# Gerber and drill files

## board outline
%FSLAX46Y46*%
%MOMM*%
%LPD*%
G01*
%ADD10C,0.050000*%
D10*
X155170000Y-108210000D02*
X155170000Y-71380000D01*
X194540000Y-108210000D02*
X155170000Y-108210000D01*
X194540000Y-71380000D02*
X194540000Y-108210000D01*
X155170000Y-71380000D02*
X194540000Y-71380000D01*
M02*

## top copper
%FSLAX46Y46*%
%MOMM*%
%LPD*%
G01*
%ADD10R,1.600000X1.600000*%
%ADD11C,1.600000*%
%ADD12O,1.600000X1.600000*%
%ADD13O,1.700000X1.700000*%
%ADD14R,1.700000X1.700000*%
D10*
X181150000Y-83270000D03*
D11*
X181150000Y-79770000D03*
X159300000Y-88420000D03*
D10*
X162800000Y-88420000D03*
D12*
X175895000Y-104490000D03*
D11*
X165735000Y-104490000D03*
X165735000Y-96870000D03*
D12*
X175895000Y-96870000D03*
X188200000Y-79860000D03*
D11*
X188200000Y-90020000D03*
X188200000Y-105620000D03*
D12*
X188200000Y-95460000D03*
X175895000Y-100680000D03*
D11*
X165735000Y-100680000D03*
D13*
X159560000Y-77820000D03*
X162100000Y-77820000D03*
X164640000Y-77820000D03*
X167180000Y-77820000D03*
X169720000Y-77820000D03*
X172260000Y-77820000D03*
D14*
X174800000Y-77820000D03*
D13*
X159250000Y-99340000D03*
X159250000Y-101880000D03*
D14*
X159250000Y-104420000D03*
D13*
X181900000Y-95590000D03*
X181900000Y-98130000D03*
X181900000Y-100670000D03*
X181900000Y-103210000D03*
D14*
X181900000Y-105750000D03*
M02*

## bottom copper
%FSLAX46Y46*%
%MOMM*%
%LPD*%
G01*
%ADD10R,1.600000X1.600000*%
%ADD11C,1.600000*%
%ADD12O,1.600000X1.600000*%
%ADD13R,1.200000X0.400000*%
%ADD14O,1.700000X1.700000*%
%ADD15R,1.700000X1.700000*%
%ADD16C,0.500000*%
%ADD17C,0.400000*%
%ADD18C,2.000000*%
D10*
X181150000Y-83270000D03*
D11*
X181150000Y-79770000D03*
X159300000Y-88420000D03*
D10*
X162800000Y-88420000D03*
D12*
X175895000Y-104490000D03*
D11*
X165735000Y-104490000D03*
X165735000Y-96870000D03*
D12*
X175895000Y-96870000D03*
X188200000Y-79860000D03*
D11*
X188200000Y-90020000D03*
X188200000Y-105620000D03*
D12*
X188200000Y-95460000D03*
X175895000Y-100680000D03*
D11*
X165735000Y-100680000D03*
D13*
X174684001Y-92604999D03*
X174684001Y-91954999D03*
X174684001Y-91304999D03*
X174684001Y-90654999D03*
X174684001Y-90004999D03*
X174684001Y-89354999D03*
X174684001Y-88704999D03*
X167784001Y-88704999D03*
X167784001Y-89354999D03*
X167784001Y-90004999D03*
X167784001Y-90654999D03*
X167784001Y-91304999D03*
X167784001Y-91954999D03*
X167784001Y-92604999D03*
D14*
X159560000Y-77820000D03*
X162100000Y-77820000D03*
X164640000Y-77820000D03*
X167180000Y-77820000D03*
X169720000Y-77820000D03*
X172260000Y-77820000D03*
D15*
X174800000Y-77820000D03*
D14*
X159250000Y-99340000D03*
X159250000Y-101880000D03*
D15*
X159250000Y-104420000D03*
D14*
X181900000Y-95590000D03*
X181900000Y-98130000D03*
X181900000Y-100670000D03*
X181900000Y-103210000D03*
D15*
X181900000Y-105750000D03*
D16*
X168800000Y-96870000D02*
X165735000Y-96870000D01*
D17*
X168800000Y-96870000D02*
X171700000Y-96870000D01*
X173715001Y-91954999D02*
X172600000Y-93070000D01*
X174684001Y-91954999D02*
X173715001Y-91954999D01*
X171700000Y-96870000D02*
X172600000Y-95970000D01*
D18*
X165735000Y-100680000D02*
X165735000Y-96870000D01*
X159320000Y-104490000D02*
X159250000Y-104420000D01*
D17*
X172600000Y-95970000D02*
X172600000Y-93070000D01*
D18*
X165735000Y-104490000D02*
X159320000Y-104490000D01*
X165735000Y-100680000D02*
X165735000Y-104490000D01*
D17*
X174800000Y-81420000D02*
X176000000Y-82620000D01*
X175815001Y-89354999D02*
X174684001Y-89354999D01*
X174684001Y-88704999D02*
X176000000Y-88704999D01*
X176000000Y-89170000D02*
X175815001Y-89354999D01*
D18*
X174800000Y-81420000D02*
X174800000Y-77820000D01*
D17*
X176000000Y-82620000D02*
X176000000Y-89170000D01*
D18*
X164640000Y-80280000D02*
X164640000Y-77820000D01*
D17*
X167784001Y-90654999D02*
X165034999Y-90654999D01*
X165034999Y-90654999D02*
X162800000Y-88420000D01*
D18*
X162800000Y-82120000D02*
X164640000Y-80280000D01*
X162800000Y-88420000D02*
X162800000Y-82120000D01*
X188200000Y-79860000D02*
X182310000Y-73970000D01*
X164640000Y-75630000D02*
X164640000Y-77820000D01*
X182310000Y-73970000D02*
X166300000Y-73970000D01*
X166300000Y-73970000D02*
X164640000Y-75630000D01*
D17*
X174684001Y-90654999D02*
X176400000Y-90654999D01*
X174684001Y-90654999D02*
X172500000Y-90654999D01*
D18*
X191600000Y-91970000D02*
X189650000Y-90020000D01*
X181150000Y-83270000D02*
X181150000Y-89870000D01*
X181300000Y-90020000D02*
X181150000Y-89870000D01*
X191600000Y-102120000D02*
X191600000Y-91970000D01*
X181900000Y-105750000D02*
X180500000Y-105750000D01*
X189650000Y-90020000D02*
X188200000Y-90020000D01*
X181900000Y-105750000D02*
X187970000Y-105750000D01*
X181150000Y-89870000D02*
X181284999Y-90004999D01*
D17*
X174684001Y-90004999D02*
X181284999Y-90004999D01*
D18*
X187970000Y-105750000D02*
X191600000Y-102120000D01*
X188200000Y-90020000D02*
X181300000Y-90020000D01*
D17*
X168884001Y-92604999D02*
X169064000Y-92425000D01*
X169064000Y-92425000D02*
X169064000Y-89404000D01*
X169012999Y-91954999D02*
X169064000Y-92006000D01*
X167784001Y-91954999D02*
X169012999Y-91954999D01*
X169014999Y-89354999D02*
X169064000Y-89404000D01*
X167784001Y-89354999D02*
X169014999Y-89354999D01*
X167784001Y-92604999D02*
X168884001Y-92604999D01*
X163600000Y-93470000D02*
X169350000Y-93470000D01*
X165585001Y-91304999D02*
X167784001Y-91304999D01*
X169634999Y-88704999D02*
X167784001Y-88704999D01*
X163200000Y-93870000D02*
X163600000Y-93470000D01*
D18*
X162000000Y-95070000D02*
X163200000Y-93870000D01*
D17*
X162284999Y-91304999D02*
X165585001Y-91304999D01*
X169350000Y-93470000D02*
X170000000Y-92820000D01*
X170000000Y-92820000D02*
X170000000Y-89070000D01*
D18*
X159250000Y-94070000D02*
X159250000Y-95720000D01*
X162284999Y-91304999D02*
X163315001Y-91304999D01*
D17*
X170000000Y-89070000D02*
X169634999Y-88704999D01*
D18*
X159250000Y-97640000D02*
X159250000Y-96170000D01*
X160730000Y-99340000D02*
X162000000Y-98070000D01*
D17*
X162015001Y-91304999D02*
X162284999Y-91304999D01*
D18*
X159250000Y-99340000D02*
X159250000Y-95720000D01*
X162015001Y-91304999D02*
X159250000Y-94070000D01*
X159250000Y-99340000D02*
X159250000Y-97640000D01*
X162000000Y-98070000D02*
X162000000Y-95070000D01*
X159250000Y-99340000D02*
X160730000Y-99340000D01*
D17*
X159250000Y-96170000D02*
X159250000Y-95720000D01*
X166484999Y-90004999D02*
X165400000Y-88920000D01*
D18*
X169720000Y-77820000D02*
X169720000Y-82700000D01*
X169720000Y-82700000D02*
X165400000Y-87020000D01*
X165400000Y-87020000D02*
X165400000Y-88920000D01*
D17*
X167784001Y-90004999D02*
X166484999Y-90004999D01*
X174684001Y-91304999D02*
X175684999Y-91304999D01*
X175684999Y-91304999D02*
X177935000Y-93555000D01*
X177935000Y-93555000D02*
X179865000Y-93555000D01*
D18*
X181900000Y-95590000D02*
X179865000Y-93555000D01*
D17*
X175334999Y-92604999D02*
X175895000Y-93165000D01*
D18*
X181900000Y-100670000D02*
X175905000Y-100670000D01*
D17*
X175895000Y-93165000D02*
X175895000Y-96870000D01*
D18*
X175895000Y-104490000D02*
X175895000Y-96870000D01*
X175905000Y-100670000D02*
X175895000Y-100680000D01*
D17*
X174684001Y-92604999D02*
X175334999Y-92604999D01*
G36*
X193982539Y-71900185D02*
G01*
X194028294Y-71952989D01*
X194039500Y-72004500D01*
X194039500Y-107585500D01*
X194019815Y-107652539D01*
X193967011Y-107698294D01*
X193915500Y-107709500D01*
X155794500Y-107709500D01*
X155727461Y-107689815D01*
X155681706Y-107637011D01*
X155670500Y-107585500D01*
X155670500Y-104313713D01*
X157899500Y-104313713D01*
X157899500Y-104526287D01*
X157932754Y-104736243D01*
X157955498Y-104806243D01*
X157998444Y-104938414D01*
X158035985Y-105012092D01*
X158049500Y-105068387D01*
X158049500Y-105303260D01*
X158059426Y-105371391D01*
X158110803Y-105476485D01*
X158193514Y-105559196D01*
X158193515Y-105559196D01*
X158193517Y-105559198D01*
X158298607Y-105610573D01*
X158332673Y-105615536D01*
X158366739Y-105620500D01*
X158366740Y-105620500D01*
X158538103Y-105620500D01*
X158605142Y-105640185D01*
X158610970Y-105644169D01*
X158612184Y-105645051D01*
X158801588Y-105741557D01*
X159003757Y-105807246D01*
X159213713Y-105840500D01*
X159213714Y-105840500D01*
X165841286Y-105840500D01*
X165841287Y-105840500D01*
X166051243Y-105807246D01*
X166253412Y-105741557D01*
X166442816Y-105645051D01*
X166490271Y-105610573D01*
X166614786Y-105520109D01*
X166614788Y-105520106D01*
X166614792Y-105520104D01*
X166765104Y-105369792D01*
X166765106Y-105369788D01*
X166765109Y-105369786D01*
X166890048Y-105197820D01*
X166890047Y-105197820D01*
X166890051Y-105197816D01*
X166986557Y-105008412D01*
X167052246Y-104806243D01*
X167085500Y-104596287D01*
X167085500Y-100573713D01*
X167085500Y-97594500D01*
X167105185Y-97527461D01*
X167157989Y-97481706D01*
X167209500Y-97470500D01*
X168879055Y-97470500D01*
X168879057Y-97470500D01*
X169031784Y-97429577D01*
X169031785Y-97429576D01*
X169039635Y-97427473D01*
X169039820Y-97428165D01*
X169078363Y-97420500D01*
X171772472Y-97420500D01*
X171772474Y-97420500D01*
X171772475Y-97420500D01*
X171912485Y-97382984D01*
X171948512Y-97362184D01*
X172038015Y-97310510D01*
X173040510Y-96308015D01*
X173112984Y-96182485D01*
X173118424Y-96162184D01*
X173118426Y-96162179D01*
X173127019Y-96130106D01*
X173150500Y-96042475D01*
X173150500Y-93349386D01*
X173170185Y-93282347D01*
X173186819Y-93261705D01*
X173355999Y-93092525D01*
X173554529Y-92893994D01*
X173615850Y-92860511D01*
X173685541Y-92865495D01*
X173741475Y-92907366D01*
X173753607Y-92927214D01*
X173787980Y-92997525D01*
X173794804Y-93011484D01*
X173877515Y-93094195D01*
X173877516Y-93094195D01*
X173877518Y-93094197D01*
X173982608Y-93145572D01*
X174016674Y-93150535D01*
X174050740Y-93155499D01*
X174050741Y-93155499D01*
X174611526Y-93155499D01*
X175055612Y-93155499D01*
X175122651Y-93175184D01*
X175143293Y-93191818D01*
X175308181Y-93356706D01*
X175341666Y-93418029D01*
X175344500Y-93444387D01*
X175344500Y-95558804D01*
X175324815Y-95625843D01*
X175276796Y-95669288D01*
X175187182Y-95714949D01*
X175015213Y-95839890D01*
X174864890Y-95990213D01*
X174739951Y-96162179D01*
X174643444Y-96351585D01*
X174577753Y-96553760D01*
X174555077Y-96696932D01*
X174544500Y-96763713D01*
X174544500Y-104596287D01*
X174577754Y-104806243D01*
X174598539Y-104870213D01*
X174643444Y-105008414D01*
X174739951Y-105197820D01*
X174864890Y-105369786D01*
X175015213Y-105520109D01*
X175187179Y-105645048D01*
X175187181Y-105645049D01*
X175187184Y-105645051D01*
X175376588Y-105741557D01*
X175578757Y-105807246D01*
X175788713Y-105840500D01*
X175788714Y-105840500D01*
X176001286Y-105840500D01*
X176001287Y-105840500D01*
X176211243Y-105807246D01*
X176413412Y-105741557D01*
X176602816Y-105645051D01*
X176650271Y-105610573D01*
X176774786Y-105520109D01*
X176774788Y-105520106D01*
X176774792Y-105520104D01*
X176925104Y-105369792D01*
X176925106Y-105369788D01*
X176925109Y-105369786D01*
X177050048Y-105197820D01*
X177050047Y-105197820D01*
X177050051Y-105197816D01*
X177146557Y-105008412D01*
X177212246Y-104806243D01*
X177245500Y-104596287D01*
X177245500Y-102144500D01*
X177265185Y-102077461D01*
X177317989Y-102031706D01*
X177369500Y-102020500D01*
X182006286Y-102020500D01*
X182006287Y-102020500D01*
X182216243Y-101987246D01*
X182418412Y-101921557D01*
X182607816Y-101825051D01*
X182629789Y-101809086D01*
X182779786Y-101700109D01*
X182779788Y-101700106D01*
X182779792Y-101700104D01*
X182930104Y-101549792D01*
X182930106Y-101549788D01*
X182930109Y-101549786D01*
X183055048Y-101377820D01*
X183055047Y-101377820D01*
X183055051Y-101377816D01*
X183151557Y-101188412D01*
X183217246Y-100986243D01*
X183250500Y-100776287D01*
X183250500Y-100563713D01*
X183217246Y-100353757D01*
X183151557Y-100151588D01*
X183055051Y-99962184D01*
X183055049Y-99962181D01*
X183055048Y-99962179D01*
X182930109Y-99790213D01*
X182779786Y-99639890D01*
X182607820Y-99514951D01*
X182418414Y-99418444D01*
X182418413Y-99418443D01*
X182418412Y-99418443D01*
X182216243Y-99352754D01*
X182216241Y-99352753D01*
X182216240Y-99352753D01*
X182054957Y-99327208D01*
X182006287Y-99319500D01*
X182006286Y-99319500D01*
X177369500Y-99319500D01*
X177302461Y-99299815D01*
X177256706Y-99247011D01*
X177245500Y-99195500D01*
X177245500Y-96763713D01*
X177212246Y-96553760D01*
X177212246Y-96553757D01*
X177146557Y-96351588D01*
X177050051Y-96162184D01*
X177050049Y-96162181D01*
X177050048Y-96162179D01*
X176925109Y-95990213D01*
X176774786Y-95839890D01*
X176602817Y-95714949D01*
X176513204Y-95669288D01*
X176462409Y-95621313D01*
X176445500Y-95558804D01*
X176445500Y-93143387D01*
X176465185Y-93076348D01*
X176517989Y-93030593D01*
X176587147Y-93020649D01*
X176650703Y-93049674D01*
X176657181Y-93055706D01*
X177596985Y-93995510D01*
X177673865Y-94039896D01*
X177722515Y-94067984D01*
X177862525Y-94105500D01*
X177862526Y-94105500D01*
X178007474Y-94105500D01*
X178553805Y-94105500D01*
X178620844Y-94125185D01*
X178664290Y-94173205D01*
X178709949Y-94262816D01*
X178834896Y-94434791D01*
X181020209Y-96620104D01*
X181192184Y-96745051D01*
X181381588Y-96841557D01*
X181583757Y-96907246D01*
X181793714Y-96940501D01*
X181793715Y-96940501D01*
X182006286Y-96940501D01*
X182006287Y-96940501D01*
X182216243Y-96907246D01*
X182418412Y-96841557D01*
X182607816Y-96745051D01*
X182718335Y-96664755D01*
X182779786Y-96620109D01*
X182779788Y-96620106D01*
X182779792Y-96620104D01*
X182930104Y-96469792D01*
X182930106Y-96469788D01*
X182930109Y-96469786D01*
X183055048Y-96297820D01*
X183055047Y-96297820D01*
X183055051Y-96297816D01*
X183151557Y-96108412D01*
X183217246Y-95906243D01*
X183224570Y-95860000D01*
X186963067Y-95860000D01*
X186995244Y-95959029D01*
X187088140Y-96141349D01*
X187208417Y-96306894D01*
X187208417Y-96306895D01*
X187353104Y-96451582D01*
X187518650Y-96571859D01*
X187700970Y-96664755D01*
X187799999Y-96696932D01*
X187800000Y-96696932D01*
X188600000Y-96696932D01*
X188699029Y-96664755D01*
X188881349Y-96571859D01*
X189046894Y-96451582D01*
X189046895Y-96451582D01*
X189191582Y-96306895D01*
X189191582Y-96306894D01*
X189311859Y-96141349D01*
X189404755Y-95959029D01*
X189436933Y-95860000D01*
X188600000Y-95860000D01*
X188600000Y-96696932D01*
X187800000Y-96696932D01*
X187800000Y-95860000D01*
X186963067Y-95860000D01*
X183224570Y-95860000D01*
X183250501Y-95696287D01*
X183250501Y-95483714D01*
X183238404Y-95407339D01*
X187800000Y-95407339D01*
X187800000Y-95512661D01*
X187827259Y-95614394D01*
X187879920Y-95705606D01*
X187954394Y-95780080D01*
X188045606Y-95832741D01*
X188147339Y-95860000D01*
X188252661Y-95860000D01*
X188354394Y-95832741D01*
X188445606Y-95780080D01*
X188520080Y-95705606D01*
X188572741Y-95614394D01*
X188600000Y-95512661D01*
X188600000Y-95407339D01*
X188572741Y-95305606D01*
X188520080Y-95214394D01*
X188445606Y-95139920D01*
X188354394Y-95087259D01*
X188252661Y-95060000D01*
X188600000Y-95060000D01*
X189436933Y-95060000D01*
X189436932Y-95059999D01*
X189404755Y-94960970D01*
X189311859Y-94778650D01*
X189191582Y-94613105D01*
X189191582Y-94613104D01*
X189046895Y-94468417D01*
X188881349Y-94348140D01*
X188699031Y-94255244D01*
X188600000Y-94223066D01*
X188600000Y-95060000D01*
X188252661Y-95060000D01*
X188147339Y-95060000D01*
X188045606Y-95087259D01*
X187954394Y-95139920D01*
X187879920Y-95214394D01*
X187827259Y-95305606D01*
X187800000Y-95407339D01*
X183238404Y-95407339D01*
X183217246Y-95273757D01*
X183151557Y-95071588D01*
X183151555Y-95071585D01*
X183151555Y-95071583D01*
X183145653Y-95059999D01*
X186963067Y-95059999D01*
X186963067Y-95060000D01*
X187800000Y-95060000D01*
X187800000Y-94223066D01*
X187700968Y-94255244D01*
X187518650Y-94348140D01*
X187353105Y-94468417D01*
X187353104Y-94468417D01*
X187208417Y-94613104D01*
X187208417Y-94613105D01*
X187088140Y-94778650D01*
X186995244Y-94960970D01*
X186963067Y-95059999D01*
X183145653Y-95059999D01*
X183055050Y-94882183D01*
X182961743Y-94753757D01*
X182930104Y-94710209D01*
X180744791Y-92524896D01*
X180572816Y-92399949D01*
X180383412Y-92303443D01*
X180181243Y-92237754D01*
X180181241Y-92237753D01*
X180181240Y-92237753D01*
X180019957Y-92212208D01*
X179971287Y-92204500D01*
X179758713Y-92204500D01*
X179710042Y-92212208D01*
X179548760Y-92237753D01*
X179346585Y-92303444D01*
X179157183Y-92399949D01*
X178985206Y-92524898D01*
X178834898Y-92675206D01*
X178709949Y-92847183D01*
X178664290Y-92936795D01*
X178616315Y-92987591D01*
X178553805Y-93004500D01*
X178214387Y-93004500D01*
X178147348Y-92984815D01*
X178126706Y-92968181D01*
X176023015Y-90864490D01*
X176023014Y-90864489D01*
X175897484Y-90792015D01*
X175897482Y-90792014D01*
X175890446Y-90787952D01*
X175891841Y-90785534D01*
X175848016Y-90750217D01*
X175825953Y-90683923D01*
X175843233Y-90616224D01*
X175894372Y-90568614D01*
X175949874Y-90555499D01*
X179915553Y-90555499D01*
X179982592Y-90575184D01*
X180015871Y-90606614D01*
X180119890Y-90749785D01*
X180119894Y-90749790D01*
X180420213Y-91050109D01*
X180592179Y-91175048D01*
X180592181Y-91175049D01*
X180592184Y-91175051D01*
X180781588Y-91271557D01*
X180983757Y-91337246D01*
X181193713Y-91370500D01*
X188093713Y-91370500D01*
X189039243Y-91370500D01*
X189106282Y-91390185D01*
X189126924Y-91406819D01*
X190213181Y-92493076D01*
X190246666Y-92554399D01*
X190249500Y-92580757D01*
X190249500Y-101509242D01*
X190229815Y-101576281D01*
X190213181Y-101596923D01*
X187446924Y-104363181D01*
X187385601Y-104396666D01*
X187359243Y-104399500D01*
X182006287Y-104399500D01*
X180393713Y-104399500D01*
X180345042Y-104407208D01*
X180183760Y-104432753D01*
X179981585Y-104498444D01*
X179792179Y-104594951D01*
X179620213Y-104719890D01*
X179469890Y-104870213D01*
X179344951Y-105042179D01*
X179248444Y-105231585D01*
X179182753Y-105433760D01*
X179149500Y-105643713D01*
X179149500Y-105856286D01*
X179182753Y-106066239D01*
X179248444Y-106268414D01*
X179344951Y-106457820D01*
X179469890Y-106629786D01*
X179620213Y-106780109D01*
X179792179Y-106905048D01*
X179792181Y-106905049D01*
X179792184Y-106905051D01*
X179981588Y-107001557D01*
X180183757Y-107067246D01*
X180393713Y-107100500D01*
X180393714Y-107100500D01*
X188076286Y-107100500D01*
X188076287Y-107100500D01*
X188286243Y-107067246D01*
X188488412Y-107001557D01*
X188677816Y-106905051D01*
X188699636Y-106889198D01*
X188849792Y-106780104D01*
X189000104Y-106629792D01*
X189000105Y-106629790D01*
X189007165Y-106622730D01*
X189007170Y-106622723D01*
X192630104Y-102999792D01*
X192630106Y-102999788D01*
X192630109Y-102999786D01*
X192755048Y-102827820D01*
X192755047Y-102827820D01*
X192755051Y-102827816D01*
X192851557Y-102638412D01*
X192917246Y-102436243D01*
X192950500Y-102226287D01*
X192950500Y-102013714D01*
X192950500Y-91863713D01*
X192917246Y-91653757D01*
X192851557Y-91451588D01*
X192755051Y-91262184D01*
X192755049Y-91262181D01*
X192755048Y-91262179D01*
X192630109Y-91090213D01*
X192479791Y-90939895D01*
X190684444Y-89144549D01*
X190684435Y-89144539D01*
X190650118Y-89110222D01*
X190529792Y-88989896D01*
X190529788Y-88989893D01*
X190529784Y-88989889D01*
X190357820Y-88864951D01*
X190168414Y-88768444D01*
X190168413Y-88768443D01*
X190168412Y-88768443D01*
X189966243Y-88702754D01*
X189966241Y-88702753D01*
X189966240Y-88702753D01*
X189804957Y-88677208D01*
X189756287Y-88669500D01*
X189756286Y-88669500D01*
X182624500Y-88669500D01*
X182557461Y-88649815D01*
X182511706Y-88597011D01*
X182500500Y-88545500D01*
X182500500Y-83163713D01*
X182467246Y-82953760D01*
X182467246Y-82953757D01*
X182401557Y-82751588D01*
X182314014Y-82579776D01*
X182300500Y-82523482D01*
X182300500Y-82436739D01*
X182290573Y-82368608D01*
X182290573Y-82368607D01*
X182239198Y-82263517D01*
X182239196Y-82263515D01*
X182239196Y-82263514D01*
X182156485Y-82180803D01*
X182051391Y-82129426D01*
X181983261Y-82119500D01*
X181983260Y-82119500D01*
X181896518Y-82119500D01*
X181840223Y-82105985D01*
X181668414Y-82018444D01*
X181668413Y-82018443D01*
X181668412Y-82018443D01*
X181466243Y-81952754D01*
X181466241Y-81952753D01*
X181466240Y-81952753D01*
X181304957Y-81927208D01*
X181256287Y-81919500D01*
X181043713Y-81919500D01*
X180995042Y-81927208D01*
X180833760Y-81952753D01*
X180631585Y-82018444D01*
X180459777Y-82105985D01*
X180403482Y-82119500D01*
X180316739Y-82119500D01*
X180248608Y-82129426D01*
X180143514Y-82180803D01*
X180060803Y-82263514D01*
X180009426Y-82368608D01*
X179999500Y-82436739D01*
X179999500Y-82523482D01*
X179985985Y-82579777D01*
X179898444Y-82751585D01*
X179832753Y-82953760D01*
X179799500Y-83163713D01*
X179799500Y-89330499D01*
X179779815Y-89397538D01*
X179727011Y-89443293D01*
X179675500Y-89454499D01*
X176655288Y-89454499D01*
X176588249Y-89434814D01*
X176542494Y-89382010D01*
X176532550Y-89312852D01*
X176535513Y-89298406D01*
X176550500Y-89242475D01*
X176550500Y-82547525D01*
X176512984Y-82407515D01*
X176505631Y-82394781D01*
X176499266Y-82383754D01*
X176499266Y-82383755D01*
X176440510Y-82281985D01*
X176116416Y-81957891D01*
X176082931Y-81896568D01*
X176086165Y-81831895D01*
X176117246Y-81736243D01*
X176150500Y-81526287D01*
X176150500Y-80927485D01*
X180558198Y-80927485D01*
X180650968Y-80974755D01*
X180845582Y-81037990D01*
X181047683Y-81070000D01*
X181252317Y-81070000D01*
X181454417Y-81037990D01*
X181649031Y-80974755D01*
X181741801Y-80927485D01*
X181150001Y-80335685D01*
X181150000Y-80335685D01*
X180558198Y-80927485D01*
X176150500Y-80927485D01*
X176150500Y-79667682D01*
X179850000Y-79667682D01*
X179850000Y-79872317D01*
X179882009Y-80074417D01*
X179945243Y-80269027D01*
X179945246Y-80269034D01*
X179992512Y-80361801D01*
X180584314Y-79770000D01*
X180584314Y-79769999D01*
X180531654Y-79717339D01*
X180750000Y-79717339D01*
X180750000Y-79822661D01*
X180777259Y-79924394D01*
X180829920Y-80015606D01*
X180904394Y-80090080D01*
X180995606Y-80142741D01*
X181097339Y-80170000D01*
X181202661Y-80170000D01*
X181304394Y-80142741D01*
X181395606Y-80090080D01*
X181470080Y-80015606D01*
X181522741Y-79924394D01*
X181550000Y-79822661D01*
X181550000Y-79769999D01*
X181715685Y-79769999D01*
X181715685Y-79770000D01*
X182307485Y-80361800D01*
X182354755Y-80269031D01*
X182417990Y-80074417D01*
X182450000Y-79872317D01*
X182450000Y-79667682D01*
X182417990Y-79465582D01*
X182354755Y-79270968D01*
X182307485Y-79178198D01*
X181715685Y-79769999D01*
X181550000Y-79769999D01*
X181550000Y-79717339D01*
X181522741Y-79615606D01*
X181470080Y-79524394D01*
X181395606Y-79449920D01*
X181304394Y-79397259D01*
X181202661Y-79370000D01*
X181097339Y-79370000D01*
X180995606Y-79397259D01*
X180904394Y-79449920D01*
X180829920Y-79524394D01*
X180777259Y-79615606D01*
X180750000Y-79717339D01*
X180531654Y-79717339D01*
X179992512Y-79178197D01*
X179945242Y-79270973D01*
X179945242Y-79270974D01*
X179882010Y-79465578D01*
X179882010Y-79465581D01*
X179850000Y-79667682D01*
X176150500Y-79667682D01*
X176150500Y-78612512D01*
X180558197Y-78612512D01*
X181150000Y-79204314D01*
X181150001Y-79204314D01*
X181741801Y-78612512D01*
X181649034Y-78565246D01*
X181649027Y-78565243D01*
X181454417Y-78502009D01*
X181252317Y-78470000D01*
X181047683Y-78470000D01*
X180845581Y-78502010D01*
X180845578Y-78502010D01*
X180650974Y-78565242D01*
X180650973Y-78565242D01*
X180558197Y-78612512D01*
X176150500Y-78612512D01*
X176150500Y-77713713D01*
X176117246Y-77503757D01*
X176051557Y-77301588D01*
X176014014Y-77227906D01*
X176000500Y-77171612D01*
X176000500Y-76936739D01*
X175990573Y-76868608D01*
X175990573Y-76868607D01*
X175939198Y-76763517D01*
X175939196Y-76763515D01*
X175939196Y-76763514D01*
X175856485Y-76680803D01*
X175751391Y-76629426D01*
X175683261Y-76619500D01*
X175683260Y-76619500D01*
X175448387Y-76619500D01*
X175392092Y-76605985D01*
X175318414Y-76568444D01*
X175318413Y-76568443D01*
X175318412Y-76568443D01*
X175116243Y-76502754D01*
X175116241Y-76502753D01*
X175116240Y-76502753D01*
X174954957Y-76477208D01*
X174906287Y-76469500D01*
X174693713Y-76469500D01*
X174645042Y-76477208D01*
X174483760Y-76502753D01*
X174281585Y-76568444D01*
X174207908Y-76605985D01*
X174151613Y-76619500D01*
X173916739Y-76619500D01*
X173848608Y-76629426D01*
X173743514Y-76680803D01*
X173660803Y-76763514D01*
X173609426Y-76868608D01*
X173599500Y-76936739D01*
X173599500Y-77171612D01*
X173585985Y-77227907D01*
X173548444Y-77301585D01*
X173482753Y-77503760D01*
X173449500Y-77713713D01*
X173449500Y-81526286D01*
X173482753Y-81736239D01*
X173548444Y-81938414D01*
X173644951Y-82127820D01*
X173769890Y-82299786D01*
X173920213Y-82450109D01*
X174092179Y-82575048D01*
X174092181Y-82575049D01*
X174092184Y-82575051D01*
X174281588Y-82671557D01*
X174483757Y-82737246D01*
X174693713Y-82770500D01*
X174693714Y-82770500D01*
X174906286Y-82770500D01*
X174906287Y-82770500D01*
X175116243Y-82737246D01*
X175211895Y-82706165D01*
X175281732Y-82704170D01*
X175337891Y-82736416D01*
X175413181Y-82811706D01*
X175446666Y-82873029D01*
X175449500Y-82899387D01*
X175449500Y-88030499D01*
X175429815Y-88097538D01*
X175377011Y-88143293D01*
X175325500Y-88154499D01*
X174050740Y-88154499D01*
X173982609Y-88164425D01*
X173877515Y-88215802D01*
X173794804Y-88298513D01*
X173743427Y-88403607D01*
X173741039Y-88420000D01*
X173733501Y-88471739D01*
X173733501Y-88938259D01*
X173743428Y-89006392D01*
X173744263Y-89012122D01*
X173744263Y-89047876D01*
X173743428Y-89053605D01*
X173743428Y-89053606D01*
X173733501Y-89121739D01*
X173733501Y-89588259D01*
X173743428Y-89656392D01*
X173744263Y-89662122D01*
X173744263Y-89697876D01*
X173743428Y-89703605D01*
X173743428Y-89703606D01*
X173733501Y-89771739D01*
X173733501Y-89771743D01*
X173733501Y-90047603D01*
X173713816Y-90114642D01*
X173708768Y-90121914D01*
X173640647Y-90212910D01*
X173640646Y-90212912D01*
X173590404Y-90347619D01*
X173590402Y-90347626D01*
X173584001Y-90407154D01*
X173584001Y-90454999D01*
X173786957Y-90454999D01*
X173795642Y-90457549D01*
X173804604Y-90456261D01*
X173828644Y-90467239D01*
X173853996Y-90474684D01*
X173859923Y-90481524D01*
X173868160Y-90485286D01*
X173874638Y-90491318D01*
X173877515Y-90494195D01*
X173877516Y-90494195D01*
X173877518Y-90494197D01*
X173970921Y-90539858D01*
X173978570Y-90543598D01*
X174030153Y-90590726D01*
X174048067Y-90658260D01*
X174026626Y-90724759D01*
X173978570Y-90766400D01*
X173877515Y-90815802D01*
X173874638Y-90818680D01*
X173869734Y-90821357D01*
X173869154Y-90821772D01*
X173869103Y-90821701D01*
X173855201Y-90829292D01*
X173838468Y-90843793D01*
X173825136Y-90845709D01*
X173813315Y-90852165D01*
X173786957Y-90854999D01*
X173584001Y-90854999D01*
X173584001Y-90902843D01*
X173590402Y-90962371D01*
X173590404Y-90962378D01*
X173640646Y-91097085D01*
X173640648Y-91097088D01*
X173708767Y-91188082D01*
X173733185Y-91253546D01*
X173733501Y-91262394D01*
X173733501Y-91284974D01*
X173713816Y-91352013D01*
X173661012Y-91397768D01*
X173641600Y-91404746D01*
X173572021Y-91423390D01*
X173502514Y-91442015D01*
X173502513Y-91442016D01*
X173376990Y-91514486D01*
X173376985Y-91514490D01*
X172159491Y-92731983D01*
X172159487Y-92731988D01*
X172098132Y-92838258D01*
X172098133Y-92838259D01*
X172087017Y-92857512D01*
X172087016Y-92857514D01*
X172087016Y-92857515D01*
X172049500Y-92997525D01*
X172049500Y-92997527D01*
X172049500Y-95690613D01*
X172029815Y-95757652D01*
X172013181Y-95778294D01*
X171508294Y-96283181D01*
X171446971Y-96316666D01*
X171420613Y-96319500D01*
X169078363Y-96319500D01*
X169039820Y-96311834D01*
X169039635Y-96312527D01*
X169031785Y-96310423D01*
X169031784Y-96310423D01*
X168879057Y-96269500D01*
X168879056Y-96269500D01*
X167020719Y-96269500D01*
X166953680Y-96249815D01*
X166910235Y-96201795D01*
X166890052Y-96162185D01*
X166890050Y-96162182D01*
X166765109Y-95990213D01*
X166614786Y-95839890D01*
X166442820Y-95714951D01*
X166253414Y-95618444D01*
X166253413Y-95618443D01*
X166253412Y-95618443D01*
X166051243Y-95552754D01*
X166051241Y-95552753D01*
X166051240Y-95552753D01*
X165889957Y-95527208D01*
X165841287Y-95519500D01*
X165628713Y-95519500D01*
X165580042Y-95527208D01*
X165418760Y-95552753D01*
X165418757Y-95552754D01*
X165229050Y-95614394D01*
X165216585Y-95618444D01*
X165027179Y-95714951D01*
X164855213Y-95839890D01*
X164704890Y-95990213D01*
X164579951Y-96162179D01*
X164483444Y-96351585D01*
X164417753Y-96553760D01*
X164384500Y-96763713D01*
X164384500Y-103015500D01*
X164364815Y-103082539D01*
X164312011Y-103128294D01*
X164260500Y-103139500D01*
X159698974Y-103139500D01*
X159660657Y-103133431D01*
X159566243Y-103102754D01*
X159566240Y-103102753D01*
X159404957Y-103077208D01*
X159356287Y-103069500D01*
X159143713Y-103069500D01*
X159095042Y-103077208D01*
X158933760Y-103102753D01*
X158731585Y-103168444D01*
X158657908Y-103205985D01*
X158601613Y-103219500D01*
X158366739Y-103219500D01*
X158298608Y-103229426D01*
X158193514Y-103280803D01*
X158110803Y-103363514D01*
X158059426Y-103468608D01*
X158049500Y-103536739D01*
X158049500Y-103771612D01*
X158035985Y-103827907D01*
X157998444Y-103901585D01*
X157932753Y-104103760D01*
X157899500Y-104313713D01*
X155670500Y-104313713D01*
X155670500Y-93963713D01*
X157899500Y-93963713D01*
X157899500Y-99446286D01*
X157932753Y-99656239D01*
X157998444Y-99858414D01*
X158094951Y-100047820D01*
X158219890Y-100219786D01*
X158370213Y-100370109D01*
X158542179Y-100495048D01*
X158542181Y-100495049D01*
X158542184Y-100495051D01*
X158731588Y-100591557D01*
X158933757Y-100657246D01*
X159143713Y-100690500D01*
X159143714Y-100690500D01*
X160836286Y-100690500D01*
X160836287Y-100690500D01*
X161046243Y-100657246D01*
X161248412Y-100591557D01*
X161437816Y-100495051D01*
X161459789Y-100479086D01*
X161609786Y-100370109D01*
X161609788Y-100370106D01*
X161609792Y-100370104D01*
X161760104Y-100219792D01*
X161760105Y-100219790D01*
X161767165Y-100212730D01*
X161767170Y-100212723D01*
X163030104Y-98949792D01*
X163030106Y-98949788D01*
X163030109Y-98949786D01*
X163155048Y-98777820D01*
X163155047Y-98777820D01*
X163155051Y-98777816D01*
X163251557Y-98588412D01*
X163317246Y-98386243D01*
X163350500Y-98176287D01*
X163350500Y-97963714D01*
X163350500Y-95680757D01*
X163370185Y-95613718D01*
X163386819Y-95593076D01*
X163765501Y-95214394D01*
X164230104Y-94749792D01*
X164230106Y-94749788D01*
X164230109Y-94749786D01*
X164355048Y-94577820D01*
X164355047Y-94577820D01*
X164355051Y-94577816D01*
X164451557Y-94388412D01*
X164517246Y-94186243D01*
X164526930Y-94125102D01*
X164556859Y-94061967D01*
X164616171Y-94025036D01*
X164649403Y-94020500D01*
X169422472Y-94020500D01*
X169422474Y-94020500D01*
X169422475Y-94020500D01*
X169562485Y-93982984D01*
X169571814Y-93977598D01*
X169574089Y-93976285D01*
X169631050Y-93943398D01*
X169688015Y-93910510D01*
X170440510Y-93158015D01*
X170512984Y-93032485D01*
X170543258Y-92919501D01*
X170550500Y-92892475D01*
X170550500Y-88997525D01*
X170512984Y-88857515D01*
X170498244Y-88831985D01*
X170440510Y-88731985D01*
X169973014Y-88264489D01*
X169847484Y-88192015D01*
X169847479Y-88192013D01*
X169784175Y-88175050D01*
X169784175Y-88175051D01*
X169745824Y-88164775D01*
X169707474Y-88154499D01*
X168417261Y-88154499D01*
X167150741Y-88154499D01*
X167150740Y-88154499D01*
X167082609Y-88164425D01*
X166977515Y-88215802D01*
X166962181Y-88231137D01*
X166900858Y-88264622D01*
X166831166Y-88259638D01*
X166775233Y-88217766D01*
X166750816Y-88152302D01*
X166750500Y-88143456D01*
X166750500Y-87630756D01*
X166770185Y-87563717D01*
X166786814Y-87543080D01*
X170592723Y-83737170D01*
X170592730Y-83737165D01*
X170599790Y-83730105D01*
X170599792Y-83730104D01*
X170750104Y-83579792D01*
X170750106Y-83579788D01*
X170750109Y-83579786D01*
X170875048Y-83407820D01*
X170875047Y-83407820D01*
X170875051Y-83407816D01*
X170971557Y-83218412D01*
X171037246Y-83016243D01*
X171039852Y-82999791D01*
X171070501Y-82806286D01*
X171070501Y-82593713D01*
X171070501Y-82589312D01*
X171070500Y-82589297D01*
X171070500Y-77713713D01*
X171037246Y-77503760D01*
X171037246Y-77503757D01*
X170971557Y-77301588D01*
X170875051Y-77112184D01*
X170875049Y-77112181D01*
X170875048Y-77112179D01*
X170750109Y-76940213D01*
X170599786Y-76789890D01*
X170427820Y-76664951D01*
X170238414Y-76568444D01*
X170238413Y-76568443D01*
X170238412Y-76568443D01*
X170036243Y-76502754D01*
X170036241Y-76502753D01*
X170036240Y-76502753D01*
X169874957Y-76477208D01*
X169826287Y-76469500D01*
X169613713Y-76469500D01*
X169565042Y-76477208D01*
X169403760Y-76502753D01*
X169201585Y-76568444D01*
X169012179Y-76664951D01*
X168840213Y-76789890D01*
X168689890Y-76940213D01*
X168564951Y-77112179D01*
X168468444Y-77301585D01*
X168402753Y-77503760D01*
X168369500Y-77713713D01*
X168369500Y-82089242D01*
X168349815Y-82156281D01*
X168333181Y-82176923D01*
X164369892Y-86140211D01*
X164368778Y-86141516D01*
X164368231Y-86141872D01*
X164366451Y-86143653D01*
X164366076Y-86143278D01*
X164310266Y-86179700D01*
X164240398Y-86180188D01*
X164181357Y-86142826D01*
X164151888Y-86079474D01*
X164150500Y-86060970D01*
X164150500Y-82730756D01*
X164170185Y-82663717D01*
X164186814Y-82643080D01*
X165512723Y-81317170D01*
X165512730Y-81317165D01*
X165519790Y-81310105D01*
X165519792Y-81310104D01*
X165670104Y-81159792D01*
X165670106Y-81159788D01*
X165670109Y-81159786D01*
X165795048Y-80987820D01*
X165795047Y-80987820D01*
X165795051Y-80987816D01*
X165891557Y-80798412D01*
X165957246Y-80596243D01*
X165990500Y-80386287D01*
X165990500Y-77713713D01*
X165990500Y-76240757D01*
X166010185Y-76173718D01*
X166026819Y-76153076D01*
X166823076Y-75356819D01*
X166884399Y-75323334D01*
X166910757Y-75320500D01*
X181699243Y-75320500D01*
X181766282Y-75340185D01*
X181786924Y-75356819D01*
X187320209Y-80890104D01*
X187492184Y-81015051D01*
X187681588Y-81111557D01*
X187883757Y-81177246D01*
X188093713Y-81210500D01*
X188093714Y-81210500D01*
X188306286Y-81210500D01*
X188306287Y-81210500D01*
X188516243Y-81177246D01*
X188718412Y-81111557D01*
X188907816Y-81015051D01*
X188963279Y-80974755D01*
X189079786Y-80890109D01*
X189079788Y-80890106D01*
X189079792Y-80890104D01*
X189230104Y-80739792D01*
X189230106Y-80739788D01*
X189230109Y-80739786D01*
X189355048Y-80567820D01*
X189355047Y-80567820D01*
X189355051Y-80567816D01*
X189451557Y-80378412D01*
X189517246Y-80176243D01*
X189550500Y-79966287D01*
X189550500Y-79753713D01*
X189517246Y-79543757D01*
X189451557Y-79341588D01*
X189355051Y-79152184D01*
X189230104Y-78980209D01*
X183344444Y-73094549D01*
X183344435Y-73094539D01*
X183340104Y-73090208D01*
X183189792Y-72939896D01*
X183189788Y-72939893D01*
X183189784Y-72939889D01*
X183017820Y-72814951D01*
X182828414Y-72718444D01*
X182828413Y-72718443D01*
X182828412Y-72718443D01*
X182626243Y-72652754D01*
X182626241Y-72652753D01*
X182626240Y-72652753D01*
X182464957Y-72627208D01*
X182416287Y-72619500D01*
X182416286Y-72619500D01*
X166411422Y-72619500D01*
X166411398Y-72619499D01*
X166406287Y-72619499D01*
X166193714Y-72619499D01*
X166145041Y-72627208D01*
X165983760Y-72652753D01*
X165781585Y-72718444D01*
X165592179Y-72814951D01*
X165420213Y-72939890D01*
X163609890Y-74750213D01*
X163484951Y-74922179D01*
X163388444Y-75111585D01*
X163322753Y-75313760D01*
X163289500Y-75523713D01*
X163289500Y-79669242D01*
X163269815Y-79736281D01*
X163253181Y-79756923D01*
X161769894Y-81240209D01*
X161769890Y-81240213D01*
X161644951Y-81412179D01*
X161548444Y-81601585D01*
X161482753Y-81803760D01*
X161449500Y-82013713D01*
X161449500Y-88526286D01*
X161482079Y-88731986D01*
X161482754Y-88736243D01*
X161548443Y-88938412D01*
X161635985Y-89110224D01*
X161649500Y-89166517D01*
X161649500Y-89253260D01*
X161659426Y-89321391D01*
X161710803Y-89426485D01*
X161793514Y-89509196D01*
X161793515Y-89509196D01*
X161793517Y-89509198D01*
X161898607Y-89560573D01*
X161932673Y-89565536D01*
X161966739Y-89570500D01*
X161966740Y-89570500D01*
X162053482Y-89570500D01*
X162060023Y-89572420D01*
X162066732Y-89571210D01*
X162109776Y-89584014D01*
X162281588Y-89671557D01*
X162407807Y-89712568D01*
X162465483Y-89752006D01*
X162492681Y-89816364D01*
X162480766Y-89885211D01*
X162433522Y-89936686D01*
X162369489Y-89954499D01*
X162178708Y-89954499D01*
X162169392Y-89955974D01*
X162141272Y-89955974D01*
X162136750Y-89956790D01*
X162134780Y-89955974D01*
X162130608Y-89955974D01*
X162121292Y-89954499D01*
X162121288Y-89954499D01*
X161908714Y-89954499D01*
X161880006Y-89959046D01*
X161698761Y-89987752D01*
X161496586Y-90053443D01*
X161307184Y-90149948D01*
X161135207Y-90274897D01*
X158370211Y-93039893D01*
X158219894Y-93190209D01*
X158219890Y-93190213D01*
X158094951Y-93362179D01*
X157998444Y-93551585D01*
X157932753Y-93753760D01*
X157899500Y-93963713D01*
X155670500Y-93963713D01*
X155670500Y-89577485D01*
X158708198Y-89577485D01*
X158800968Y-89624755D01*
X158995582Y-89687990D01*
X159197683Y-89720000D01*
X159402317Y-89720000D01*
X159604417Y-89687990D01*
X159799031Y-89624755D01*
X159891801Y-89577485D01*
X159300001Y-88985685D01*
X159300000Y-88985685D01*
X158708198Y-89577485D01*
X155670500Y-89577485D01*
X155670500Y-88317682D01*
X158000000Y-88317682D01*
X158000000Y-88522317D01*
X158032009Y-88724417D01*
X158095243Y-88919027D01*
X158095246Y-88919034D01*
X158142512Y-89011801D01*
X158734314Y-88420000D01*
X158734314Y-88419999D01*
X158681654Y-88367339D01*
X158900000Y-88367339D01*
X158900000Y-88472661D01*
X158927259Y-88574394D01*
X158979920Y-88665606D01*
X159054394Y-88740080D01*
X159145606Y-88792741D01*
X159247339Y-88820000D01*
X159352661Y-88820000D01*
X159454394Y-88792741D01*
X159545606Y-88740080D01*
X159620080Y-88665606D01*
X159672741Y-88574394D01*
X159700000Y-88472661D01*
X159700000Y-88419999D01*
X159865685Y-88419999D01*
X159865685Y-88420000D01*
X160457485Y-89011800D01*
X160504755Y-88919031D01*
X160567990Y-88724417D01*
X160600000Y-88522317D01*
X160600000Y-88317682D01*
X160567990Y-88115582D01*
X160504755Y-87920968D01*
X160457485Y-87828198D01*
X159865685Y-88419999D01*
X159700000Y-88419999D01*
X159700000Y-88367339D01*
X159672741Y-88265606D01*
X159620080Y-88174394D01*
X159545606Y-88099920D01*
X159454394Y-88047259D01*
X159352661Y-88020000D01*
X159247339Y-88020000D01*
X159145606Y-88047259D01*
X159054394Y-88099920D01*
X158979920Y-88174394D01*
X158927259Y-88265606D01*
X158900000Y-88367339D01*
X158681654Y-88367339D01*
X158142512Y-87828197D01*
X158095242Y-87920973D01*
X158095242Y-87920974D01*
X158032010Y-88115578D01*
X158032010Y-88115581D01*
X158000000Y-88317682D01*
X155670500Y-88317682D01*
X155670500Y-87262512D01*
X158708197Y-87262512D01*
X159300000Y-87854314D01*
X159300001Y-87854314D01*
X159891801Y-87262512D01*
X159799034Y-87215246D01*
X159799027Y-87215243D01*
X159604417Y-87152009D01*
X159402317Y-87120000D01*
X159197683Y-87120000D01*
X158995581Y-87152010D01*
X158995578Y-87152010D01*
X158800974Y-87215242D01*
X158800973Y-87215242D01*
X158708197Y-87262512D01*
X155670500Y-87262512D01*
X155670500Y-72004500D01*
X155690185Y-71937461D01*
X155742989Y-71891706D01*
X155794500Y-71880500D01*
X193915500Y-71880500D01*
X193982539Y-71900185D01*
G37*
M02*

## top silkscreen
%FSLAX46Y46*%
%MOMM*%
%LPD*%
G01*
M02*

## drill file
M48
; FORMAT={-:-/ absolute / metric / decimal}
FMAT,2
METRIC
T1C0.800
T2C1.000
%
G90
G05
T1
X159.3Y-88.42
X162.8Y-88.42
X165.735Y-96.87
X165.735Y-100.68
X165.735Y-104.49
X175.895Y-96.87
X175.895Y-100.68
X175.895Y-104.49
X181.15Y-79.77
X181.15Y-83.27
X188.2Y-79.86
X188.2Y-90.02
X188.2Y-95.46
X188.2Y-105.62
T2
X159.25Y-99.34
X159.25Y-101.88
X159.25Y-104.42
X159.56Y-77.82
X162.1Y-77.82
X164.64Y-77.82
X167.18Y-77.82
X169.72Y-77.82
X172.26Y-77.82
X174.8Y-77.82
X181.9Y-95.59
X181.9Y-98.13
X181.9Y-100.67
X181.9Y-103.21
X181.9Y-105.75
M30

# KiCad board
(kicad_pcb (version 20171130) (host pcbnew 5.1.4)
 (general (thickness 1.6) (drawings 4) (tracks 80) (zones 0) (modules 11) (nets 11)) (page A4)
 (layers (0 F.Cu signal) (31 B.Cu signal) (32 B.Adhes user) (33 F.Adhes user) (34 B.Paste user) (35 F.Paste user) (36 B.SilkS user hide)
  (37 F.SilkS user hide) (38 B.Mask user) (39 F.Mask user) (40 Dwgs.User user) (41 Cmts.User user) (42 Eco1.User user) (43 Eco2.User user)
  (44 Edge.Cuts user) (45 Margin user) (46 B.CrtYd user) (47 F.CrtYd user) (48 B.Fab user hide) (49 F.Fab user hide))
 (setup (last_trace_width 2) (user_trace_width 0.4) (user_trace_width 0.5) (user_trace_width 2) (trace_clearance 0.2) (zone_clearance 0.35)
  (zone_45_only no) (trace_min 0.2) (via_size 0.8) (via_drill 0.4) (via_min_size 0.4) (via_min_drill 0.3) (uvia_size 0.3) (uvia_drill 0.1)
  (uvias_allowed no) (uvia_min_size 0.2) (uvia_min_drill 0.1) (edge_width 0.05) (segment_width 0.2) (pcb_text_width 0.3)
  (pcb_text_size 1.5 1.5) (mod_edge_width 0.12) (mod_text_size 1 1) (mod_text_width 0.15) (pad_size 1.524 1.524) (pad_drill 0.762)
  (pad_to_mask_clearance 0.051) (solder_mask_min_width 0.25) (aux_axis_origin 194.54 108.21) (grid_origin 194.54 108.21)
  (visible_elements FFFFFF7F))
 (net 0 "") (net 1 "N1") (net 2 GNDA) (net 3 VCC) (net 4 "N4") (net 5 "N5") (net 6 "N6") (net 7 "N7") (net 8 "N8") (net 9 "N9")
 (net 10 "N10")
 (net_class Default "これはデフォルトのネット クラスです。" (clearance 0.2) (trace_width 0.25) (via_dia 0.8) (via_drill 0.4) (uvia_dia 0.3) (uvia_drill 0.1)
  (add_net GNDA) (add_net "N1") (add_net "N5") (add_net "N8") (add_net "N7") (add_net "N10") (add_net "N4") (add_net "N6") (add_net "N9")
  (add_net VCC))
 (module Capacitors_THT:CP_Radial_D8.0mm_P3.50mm (layer B.Cu) (at 181.15 83.27 90)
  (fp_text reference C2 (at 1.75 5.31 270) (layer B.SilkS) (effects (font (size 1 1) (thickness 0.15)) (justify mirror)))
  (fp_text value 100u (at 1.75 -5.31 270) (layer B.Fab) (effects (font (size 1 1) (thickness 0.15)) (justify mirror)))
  (pad 1 thru_hole rect (at 0 0 90) (size 1.6 1.6) (drill 0.8) (layers *.Cu *.Mask) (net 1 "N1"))
  (pad 2 thru_hole circle (at 3.5 0 90) (size 1.6 1.6) (drill 0.8) (layers *.Cu *.Mask) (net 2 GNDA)))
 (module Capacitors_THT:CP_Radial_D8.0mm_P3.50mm (layer B.Cu) (at 162.8 88.42 180)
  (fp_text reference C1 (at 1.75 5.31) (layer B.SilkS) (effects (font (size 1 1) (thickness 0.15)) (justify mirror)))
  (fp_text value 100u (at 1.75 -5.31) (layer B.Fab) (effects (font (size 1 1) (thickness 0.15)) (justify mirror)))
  (pad 2 thru_hole circle (at 3.5 0 180) (size 1.6 1.6) (drill 0.8) (layers *.Cu *.Mask) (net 2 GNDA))
  (pad 1 thru_hole rect (at 0 0 180) (size 1.6 1.6) (drill 0.8) (layers *.Cu *.Mask) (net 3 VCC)))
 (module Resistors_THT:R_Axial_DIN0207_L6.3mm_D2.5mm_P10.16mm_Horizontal (layer B.Cu) (at 165.735 104.49)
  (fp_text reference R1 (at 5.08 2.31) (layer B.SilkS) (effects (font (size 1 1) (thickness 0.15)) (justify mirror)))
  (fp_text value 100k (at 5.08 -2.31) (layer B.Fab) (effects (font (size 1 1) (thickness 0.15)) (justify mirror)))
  (pad 2 thru_hole oval (at 10.16 0) (size 1.6 1.6) (drill 0.8) (layers *.Cu *.Mask) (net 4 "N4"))
  (pad 1 thru_hole circle (at 0 0) (size 1.6 1.6) (drill 0.8) (layers *.Cu *.Mask) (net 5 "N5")))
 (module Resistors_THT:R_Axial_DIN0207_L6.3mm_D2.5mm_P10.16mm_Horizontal (layer B.Cu) (at 165.735 96.87)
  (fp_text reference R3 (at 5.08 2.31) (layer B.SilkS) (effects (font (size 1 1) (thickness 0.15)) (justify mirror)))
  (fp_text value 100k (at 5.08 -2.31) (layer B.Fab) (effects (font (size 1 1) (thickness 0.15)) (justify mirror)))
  (pad 1 thru_hole circle (at 0 0) (size 1.6 1.6) (drill 0.8) (layers *.Cu *.Mask) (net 5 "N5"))
  (pad 2 thru_hole oval (at 10.16 0) (size 1.6 1.6) (drill 0.8) (layers *.Cu *.Mask) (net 4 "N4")))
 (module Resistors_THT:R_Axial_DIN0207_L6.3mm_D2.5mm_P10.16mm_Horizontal (layer B.Cu) (at 188.2 90.02 90)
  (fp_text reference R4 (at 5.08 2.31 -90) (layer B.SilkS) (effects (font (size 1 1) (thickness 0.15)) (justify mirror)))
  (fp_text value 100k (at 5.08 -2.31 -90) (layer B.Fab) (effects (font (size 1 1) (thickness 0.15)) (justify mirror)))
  (pad 2 thru_hole oval (at 10.16 0 90) (size 1.6 1.6) (drill 0.8) (layers *.Cu *.Mask) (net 3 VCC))
  (pad 1 thru_hole circle (at 0 0 90) (size 1.6 1.6) (drill 0.8) (layers *.Cu *.Mask) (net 1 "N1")))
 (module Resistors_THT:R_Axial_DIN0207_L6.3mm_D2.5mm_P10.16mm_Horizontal (layer B.Cu) (at 188.2 105.62 90)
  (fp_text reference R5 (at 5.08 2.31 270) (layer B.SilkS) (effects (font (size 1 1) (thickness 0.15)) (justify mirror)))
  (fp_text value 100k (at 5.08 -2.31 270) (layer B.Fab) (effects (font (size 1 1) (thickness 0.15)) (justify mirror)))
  (pad 1 thru_hole circle (at 0 0 90) (size 1.6 1.6) (drill 0.8) (layers *.Cu *.Mask) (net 1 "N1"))
  (pad 2 thru_hole oval (at 10.16 0 90) (size 1.6 1.6) (drill 0.8) (layers *.Cu *.Mask) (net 2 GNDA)))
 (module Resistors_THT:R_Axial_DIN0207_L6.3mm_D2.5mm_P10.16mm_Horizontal (layer B.Cu) (at 165.735 100.68)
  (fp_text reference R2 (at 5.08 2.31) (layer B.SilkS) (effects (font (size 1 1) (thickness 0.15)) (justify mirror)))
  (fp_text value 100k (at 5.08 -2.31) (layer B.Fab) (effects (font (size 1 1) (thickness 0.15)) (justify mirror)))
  (pad 2 thru_hole oval (at 10.16 0) (size 1.6 1.6) (drill 0.8) (layers *.Cu *.Mask) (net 4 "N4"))
  (pad 1 thru_hole circle (at 0 0) (size 1.6 1.6) (drill 0.8) (layers *.Cu *.Mask) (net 5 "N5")))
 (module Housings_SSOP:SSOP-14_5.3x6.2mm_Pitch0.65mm (layer B.Cu) (at 171.234001 90.654999)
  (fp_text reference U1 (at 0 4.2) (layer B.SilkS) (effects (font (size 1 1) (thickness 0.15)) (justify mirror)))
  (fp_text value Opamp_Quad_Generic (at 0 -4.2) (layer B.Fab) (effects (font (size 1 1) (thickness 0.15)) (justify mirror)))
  (pad 14 smd rect (at 3.45 1.95) (size 1.2 0.4) (layers B.Cu B.Paste B.Mask) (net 4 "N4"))
  (pad 13 smd rect (at 3.45 1.3) (size 1.2 0.4) (layers B.Cu B.Paste B.Mask) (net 5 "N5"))
  (pad 12 smd rect (at 3.45 0.65) (size 1.2 0.4) (layers B.Cu B.Paste B.Mask) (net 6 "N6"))
  (pad 11 smd rect (at 3.45 0) (size 1.2 0.4) (layers B.Cu B.Paste B.Mask) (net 2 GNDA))
  (pad 10 smd rect (at 3.45 -0.65) (size 1.2 0.4) (layers B.Cu B.Paste B.Mask) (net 1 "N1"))
  (pad 9 smd rect (at 3.45 -1.3) (size 1.2 0.4) (layers B.Cu B.Paste B.Mask) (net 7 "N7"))
  (pad 8 smd rect (at 3.45 -1.95) (size 1.2 0.4) (layers B.Cu B.Paste B.Mask) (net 7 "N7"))
  (pad 7 smd rect (at -3.45 -1.95) (size 1.2 0.4) (layers B.Cu B.Paste B.Mask) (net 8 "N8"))
  (pad 6 smd rect (at -3.45 -1.3) (size 1.2 0.4) (layers B.Cu B.Paste B.Mask) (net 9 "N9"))
  (pad 5 smd rect (at -3.45 -0.65) (size 1.2 0.4) (layers B.Cu B.Paste B.Mask) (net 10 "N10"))
  (pad 4 smd rect (at -3.45 0) (size 1.2 0.4) (layers B.Cu B.Paste B.Mask) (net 3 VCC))
  (pad 3 smd rect (at -3.45 0.65) (size 1.2 0.4) (layers B.Cu B.Paste B.Mask) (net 8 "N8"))
  (pad 2 smd rect (at -3.45 1.3) (size 1.2 0.4) (layers B.Cu B.Paste B.Mask) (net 9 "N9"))
  (pad 1 smd rect (at -3.45 1.95) (size 1.2 0.4) (layers B.Cu B.Paste B.Mask) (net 9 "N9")))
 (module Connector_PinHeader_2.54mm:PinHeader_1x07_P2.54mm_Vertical (layer B.Cu) (at 174.8 77.82 90) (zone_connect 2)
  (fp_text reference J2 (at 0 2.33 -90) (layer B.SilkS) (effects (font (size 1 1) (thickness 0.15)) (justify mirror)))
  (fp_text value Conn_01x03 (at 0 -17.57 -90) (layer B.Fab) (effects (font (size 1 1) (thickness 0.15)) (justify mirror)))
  (pad 7 thru_hole oval (at 0 -15.24 90) (size 1.7 1.7) (drill 1) (layers *.Cu *.Mask) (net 2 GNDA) (zone_connect 2))
  (pad 6 thru_hole oval (at 0 -12.7 90) (size 1.7 1.7) (drill 1) (layers *.Cu *.Mask) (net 2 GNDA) (zone_connect 2))
  (pad 5 thru_hole oval (at 0 -10.16 90) (size 1.7 1.7) (drill 1) (layers *.Cu *.Mask) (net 3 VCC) (zone_connect 2))
  (pad 4 thru_hole oval (at 0 -7.62 90) (size 1.7 1.7) (drill 1) (layers *.Cu *.Mask) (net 2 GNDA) (zone_connect 2))
  (pad 3 thru_hole oval (at 0 -5.08 90) (size 1.7 1.7) (drill 1) (layers *.Cu *.Mask) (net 10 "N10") (zone_connect 2))
  (pad 2 thru_hole oval (at 0 -2.54 90) (size 1.7 1.7) (drill 1) (layers *.Cu *.Mask) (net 2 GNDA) (zone_connect 2))
  (pad 1 thru_hole rect (at 0 0 90) (size 1.7 1.7) (drill 1) (layers *.Cu *.Mask) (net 7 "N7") (zone_connect 2)))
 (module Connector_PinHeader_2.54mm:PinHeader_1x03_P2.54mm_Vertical (layer B.Cu) (at 159.25 104.42) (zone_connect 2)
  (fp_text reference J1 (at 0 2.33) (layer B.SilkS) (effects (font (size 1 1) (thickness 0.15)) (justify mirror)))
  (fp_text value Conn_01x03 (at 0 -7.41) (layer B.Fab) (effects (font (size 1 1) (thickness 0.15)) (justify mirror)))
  (pad 3 thru_hole oval (at 0 -5.08) (size 1.7 1.7) (drill 1) (layers *.Cu *.Mask) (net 8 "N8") (zone_connect 2))
  (pad 2 thru_hole oval (at 0 -2.54) (size 1.7 1.7) (drill 1) (layers *.Cu *.Mask) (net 2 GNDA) (zone_connect 2))
  (pad 1 thru_hole rect (at 0 0) (size 1.7 1.7) (drill 1) (layers *.Cu *.Mask) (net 5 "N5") (zone_connect 2)))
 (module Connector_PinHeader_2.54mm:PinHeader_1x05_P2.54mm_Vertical (layer B.Cu) (at 181.9 105.75) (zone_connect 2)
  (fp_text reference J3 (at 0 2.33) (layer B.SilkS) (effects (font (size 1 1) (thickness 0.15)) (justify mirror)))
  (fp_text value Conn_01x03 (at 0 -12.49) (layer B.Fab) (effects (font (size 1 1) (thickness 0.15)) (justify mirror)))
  (pad 5 thru_hole oval (at 0 -10.16) (size 1.7 1.7) (drill 1) (layers *.Cu *.Mask) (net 6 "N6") (zone_connect 2))
  (pad 4 thru_hole oval (at 0 -7.62) (size 1.7 1.7) (drill 1) (layers *.Cu *.Mask) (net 2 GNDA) (zone_connect 2))
  (pad 3 thru_hole oval (at 0 -5.08) (size 1.7 1.7) (drill 1) (layers *.Cu *.Mask) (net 4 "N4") (zone_connect 2))
  (pad 2 thru_hole oval (at 0 -2.54) (size 1.7 1.7) (drill 1) (layers *.Cu *.Mask) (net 2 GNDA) (zone_connect 2))
  (pad 1 thru_hole rect (at 0 0) (size 1.7 1.7) (drill 1) (layers *.Cu *.Mask) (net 1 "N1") (zone_connect 2)))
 (gr_line (start 155.17 108.21) (end 155.17 71.38) (layer Edge.Cuts) (width 0.05))
 (gr_line (start 194.54 108.21) (end 155.17 108.21) (layer Edge.Cuts) (width 0.05))
 (gr_line (start 194.54 71.38) (end 194.54 108.21) (layer Edge.Cuts) (width 0.05))
 (gr_line (start 155.17 71.38) (end 194.54 71.38) (layer Edge.Cuts) (width 0.05))
 (segment (start 168.8 96.87) (end 165.735 96.87) (width 0.5) (layer B.Cu) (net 5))
 (segment (start 168.8 96.87) (end 171.7 96.87) (width 0.4) (layer B.Cu) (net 5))
 (segment (start 173.715001 91.954999) (end 172.6 93.07) (width 0.4) (layer B.Cu) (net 5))
 (segment (start 174.684001 91.954999) (end 173.715001 91.954999) (width 0.4) (layer B.Cu) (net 5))
 (segment (start 171.7 96.87) (end 172.6 95.97) (width 0.4) (layer B.Cu) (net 5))
 (segment (start 165.735 100.68) (end 165.735 96.87) (width 2) (layer B.Cu) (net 5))
 (segment (start 159.32 104.49) (end 159.25 104.42) (width 2) (layer B.Cu) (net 5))
 (segment (start 172.6 95.97) (end 172.6 93.07) (width 0.4) (layer B.Cu) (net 5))
 (segment (start 165.735 104.49) (end 159.32 104.49) (width 2) (layer B.Cu) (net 5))
 (segment (start 165.735 100.68) (end 165.735 104.49) (width 2) (layer B.Cu) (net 5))
 (segment (start 174.8 81.42) (end 176 82.62) (width 0.4) (layer B.Cu) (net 7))
 (segment (start 175.815001 89.354999) (end 174.684001 89.354999) (width 0.4) (layer B.Cu) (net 7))
 (segment (start 174.684001 88.704999) (end 176 88.704999) (width 0.4) (layer B.Cu) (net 7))
 (segment (start 176 89.17) (end 175.815001 89.354999) (width 0.4) (layer B.Cu) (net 7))
 (segment (start 174.8 81.42) (end 174.8 77.82) (width 2) (layer B.Cu) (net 7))
 (segment (start 176 82.62) (end 176 89.17) (width 0.4) (layer B.Cu) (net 7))
 (segment (start 164.64 80.28) (end 164.64 77.82) (width 2) (layer B.Cu) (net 3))
 (segment (start 167.784001 90.654999) (end 165.034999 90.654999) (width 0.4) (layer B.Cu) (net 3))
 (segment (start 165.034999 90.654999) (end 162.8 88.42) (width 0.4) (layer B.Cu) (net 3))
 (segment (start 162.8 82.12) (end 164.64 80.28) (width 2) (layer B.Cu) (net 3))
 (segment (start 162.8 88.42) (end 162.8 82.12) (width 2) (layer B.Cu) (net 3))
 (segment (start 188.2 79.86) (end 182.31 73.97) (width 2) (layer B.Cu) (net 3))
 (segment (start 164.64 75.63) (end 164.64 77.82) (width 2) (layer B.Cu) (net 3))
 (segment (start 182.31 73.97) (end 166.3 73.97) (width 2) (layer B.Cu) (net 3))
 (segment (start 166.3 73.97) (end 164.64 75.63) (width 2) (layer B.Cu) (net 3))
 (segment (start 174.684001 90.654999) (end 176.4 90.654999) (width 0.4) (layer B.Cu) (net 2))
 (segment (start 174.684001 90.654999) (end 172.5 90.654999) (width 0.4) (layer B.Cu) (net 2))
 (segment (start 191.6 91.97) (end 189.65 90.02) (width 2) (layer B.Cu) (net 1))
 (segment (start 181.15 83.27) (end 181.15 89.87) (width 2) (layer B.Cu) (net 1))
 (segment (start 181.3 90.02) (end 181.15 89.87) (width 2) (layer B.Cu) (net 1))
 (segment (start 191.6 102.12) (end 191.6 91.97) (width 2) (layer B.Cu) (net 1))
 (segment (start 181.9 105.75) (end 180.5 105.75) (width 2) (layer B.Cu) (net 1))
 (segment (start 189.65 90.02) (end 188.2 90.02) (width 2) (layer B.Cu) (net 1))
 (segment (start 181.9 105.75) (end 187.97 105.75) (width 2) (layer B.Cu) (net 1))
 (segment (start 181.15 89.87) (end 181.284999 90.004999) (width 2) (layer B.Cu) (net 1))
 (segment (start 174.684001 90.004999) (end 181.284999 90.004999) (width 0.4) (layer B.Cu) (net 1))
 (segment (start 187.97 105.75) (end 191.6 102.12) (width 2) (layer B.Cu) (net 1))
 (segment (start 188.2 90.02) (end 181.3 90.02) (width 2) (layer B.Cu) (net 1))
 (segment (start 168.884001 92.604999) (end 169.064 92.425) (width 0.4) (layer B.Cu) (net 9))
 (segment (start 169.064 92.425) (end 169.064 89.404) (width 0.4) (layer B.Cu) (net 9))
 (segment (start 169.012999 91.954999) (end 169.064 92.006) (width 0.4) (layer B.Cu) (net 9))
 (segment (start 167.784001 91.954999) (end 169.012999 91.954999) (width 0.4) (layer B.Cu) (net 9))
 (segment (start 169.014999 89.354999) (end 169.064 89.404) (width 0.4) (layer B.Cu) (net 9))
 (segment (start 167.784001 89.354999) (end 169.014999 89.354999) (width 0.4) (layer B.Cu) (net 9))
 (segment (start 167.784001 92.604999) (end 168.884001 92.604999) (width 0.4) (layer B.Cu) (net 9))
 (segment (start 163.6 93.47) (end 169.35 93.47) (width 0.4) (layer B.Cu) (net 8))
 (segment (start 165.585001 91.304999) (end 167.784001 91.304999) (width 0.4) (layer B.Cu) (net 8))
 (segment (start 169.634999 88.704999) (end 167.784001 88.704999) (width 0.4) (layer B.Cu) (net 8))
 (segment (start 163.2 93.87) (end 163.6 93.47) (width 0.4) (layer B.Cu) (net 8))
 (segment (start 162 95.07) (end 163.2 93.87) (width 2) (layer B.Cu) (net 8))
 (segment (start 162.284999 91.304999) (end 165.585001 91.304999) (width 0.4) (layer B.Cu) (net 8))
 (segment (start 169.35 93.47) (end 170 92.82) (width 0.4) (layer B.Cu) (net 8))
 (segment (start 170 92.82) (end 170 89.07) (width 0.4) (layer B.Cu) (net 8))
 (segment (start 159.25 94.07) (end 159.25 95.72) (width 2) (layer B.Cu) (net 8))
 (segment (start 162.284999 91.304999) (end 163.315001 91.304999) (width 2) (layer B.Cu) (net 8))
 (segment (start 170 89.07) (end 169.634999 88.704999) (width 0.4) (layer B.Cu) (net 8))
 (segment (start 159.25 97.64) (end 159.25 96.17) (width 2) (layer B.Cu) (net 8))
 (segment (start 160.73 99.34) (end 162 98.07) (width 2) (layer B.Cu) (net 8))
 (segment (start 162.015001 91.304999) (end 162.284999 91.304999) (width 0.4) (layer B.Cu) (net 8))
 (segment (start 159.25 99.34) (end 159.25 95.72) (width 2) (layer B.Cu) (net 8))
 (segment (start 162.015001 91.304999) (end 159.25 94.07) (width 2) (layer B.Cu) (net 8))
 (segment (start 159.25 99.34) (end 159.25 97.64) (width 2) (layer B.Cu) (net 8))
 (segment (start 162 98.07) (end 162 95.07) (width 2) (layer B.Cu) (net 8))
 (segment (start 159.25 99.34) (end 160.73 99.34) (width 2) (layer B.Cu) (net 8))
 (segment (start 159.25 96.17) (end 159.25 95.72) (width 0.4) (layer B.Cu) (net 8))
 (segment (start 166.484999 90.004999) (end 165.4 88.92) (width 0.4) (layer B.Cu) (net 10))
 (segment (start 169.72 77.82) (end 169.72 82.7) (width 2) (layer B.Cu) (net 10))
 (segment (start 169.72 82.7) (end 165.4 87.02) (width 2) (layer B.Cu) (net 10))
 (segment (start 165.4 87.02) (end 165.4 88.92) (width 2) (layer B.Cu) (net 10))
 (segment (start 167.784001 90.004999) (end 166.484999 90.004999) (width 0.4) (layer B.Cu) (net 10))
 (segment (start 174.684001 91.304999) (end 175.684999 91.304999) (width 0.4) (layer B.Cu) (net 6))
 (segment (start 175.684999 91.304999) (end 177.935 93.555) (width 0.4) (layer B.Cu) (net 6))
 (segment (start 177.935 93.555) (end 179.865 93.555) (width 0.4) (layer B.Cu) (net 6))
 (segment (start 181.9 95.59) (end 179.865 93.555) (width 2) (layer B.Cu) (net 6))
 (segment (start 175.334999 92.604999) (end 175.895 93.165) (width 0.4) (layer B.Cu) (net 4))
 (segment (start 181.9 100.67) (end 175.905 100.67) (width 2) (layer B.Cu) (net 4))
 (segment (start 175.895 93.165) (end 175.895 96.87) (width 0.4) (layer B.Cu) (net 4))
 (segment (start 175.895 104.49) (end 175.895 96.87) (width 2) (layer B.Cu) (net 4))
 (segment (start 175.905 100.67) (end 175.895 100.68) (width 2) (layer B.Cu) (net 4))
 (segment (start 174.684001 92.604999) (end 175.334999 92.604999) (width 0.4) (layer B.Cu) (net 4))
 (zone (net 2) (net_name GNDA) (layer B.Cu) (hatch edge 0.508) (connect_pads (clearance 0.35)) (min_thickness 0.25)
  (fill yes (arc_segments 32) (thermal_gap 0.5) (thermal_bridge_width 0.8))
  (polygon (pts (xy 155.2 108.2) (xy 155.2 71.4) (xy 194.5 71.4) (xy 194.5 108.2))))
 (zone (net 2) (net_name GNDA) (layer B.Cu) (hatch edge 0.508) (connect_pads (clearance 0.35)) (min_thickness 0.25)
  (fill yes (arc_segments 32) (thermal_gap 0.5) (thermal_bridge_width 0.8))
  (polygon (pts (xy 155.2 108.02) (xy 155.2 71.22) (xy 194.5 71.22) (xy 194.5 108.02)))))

